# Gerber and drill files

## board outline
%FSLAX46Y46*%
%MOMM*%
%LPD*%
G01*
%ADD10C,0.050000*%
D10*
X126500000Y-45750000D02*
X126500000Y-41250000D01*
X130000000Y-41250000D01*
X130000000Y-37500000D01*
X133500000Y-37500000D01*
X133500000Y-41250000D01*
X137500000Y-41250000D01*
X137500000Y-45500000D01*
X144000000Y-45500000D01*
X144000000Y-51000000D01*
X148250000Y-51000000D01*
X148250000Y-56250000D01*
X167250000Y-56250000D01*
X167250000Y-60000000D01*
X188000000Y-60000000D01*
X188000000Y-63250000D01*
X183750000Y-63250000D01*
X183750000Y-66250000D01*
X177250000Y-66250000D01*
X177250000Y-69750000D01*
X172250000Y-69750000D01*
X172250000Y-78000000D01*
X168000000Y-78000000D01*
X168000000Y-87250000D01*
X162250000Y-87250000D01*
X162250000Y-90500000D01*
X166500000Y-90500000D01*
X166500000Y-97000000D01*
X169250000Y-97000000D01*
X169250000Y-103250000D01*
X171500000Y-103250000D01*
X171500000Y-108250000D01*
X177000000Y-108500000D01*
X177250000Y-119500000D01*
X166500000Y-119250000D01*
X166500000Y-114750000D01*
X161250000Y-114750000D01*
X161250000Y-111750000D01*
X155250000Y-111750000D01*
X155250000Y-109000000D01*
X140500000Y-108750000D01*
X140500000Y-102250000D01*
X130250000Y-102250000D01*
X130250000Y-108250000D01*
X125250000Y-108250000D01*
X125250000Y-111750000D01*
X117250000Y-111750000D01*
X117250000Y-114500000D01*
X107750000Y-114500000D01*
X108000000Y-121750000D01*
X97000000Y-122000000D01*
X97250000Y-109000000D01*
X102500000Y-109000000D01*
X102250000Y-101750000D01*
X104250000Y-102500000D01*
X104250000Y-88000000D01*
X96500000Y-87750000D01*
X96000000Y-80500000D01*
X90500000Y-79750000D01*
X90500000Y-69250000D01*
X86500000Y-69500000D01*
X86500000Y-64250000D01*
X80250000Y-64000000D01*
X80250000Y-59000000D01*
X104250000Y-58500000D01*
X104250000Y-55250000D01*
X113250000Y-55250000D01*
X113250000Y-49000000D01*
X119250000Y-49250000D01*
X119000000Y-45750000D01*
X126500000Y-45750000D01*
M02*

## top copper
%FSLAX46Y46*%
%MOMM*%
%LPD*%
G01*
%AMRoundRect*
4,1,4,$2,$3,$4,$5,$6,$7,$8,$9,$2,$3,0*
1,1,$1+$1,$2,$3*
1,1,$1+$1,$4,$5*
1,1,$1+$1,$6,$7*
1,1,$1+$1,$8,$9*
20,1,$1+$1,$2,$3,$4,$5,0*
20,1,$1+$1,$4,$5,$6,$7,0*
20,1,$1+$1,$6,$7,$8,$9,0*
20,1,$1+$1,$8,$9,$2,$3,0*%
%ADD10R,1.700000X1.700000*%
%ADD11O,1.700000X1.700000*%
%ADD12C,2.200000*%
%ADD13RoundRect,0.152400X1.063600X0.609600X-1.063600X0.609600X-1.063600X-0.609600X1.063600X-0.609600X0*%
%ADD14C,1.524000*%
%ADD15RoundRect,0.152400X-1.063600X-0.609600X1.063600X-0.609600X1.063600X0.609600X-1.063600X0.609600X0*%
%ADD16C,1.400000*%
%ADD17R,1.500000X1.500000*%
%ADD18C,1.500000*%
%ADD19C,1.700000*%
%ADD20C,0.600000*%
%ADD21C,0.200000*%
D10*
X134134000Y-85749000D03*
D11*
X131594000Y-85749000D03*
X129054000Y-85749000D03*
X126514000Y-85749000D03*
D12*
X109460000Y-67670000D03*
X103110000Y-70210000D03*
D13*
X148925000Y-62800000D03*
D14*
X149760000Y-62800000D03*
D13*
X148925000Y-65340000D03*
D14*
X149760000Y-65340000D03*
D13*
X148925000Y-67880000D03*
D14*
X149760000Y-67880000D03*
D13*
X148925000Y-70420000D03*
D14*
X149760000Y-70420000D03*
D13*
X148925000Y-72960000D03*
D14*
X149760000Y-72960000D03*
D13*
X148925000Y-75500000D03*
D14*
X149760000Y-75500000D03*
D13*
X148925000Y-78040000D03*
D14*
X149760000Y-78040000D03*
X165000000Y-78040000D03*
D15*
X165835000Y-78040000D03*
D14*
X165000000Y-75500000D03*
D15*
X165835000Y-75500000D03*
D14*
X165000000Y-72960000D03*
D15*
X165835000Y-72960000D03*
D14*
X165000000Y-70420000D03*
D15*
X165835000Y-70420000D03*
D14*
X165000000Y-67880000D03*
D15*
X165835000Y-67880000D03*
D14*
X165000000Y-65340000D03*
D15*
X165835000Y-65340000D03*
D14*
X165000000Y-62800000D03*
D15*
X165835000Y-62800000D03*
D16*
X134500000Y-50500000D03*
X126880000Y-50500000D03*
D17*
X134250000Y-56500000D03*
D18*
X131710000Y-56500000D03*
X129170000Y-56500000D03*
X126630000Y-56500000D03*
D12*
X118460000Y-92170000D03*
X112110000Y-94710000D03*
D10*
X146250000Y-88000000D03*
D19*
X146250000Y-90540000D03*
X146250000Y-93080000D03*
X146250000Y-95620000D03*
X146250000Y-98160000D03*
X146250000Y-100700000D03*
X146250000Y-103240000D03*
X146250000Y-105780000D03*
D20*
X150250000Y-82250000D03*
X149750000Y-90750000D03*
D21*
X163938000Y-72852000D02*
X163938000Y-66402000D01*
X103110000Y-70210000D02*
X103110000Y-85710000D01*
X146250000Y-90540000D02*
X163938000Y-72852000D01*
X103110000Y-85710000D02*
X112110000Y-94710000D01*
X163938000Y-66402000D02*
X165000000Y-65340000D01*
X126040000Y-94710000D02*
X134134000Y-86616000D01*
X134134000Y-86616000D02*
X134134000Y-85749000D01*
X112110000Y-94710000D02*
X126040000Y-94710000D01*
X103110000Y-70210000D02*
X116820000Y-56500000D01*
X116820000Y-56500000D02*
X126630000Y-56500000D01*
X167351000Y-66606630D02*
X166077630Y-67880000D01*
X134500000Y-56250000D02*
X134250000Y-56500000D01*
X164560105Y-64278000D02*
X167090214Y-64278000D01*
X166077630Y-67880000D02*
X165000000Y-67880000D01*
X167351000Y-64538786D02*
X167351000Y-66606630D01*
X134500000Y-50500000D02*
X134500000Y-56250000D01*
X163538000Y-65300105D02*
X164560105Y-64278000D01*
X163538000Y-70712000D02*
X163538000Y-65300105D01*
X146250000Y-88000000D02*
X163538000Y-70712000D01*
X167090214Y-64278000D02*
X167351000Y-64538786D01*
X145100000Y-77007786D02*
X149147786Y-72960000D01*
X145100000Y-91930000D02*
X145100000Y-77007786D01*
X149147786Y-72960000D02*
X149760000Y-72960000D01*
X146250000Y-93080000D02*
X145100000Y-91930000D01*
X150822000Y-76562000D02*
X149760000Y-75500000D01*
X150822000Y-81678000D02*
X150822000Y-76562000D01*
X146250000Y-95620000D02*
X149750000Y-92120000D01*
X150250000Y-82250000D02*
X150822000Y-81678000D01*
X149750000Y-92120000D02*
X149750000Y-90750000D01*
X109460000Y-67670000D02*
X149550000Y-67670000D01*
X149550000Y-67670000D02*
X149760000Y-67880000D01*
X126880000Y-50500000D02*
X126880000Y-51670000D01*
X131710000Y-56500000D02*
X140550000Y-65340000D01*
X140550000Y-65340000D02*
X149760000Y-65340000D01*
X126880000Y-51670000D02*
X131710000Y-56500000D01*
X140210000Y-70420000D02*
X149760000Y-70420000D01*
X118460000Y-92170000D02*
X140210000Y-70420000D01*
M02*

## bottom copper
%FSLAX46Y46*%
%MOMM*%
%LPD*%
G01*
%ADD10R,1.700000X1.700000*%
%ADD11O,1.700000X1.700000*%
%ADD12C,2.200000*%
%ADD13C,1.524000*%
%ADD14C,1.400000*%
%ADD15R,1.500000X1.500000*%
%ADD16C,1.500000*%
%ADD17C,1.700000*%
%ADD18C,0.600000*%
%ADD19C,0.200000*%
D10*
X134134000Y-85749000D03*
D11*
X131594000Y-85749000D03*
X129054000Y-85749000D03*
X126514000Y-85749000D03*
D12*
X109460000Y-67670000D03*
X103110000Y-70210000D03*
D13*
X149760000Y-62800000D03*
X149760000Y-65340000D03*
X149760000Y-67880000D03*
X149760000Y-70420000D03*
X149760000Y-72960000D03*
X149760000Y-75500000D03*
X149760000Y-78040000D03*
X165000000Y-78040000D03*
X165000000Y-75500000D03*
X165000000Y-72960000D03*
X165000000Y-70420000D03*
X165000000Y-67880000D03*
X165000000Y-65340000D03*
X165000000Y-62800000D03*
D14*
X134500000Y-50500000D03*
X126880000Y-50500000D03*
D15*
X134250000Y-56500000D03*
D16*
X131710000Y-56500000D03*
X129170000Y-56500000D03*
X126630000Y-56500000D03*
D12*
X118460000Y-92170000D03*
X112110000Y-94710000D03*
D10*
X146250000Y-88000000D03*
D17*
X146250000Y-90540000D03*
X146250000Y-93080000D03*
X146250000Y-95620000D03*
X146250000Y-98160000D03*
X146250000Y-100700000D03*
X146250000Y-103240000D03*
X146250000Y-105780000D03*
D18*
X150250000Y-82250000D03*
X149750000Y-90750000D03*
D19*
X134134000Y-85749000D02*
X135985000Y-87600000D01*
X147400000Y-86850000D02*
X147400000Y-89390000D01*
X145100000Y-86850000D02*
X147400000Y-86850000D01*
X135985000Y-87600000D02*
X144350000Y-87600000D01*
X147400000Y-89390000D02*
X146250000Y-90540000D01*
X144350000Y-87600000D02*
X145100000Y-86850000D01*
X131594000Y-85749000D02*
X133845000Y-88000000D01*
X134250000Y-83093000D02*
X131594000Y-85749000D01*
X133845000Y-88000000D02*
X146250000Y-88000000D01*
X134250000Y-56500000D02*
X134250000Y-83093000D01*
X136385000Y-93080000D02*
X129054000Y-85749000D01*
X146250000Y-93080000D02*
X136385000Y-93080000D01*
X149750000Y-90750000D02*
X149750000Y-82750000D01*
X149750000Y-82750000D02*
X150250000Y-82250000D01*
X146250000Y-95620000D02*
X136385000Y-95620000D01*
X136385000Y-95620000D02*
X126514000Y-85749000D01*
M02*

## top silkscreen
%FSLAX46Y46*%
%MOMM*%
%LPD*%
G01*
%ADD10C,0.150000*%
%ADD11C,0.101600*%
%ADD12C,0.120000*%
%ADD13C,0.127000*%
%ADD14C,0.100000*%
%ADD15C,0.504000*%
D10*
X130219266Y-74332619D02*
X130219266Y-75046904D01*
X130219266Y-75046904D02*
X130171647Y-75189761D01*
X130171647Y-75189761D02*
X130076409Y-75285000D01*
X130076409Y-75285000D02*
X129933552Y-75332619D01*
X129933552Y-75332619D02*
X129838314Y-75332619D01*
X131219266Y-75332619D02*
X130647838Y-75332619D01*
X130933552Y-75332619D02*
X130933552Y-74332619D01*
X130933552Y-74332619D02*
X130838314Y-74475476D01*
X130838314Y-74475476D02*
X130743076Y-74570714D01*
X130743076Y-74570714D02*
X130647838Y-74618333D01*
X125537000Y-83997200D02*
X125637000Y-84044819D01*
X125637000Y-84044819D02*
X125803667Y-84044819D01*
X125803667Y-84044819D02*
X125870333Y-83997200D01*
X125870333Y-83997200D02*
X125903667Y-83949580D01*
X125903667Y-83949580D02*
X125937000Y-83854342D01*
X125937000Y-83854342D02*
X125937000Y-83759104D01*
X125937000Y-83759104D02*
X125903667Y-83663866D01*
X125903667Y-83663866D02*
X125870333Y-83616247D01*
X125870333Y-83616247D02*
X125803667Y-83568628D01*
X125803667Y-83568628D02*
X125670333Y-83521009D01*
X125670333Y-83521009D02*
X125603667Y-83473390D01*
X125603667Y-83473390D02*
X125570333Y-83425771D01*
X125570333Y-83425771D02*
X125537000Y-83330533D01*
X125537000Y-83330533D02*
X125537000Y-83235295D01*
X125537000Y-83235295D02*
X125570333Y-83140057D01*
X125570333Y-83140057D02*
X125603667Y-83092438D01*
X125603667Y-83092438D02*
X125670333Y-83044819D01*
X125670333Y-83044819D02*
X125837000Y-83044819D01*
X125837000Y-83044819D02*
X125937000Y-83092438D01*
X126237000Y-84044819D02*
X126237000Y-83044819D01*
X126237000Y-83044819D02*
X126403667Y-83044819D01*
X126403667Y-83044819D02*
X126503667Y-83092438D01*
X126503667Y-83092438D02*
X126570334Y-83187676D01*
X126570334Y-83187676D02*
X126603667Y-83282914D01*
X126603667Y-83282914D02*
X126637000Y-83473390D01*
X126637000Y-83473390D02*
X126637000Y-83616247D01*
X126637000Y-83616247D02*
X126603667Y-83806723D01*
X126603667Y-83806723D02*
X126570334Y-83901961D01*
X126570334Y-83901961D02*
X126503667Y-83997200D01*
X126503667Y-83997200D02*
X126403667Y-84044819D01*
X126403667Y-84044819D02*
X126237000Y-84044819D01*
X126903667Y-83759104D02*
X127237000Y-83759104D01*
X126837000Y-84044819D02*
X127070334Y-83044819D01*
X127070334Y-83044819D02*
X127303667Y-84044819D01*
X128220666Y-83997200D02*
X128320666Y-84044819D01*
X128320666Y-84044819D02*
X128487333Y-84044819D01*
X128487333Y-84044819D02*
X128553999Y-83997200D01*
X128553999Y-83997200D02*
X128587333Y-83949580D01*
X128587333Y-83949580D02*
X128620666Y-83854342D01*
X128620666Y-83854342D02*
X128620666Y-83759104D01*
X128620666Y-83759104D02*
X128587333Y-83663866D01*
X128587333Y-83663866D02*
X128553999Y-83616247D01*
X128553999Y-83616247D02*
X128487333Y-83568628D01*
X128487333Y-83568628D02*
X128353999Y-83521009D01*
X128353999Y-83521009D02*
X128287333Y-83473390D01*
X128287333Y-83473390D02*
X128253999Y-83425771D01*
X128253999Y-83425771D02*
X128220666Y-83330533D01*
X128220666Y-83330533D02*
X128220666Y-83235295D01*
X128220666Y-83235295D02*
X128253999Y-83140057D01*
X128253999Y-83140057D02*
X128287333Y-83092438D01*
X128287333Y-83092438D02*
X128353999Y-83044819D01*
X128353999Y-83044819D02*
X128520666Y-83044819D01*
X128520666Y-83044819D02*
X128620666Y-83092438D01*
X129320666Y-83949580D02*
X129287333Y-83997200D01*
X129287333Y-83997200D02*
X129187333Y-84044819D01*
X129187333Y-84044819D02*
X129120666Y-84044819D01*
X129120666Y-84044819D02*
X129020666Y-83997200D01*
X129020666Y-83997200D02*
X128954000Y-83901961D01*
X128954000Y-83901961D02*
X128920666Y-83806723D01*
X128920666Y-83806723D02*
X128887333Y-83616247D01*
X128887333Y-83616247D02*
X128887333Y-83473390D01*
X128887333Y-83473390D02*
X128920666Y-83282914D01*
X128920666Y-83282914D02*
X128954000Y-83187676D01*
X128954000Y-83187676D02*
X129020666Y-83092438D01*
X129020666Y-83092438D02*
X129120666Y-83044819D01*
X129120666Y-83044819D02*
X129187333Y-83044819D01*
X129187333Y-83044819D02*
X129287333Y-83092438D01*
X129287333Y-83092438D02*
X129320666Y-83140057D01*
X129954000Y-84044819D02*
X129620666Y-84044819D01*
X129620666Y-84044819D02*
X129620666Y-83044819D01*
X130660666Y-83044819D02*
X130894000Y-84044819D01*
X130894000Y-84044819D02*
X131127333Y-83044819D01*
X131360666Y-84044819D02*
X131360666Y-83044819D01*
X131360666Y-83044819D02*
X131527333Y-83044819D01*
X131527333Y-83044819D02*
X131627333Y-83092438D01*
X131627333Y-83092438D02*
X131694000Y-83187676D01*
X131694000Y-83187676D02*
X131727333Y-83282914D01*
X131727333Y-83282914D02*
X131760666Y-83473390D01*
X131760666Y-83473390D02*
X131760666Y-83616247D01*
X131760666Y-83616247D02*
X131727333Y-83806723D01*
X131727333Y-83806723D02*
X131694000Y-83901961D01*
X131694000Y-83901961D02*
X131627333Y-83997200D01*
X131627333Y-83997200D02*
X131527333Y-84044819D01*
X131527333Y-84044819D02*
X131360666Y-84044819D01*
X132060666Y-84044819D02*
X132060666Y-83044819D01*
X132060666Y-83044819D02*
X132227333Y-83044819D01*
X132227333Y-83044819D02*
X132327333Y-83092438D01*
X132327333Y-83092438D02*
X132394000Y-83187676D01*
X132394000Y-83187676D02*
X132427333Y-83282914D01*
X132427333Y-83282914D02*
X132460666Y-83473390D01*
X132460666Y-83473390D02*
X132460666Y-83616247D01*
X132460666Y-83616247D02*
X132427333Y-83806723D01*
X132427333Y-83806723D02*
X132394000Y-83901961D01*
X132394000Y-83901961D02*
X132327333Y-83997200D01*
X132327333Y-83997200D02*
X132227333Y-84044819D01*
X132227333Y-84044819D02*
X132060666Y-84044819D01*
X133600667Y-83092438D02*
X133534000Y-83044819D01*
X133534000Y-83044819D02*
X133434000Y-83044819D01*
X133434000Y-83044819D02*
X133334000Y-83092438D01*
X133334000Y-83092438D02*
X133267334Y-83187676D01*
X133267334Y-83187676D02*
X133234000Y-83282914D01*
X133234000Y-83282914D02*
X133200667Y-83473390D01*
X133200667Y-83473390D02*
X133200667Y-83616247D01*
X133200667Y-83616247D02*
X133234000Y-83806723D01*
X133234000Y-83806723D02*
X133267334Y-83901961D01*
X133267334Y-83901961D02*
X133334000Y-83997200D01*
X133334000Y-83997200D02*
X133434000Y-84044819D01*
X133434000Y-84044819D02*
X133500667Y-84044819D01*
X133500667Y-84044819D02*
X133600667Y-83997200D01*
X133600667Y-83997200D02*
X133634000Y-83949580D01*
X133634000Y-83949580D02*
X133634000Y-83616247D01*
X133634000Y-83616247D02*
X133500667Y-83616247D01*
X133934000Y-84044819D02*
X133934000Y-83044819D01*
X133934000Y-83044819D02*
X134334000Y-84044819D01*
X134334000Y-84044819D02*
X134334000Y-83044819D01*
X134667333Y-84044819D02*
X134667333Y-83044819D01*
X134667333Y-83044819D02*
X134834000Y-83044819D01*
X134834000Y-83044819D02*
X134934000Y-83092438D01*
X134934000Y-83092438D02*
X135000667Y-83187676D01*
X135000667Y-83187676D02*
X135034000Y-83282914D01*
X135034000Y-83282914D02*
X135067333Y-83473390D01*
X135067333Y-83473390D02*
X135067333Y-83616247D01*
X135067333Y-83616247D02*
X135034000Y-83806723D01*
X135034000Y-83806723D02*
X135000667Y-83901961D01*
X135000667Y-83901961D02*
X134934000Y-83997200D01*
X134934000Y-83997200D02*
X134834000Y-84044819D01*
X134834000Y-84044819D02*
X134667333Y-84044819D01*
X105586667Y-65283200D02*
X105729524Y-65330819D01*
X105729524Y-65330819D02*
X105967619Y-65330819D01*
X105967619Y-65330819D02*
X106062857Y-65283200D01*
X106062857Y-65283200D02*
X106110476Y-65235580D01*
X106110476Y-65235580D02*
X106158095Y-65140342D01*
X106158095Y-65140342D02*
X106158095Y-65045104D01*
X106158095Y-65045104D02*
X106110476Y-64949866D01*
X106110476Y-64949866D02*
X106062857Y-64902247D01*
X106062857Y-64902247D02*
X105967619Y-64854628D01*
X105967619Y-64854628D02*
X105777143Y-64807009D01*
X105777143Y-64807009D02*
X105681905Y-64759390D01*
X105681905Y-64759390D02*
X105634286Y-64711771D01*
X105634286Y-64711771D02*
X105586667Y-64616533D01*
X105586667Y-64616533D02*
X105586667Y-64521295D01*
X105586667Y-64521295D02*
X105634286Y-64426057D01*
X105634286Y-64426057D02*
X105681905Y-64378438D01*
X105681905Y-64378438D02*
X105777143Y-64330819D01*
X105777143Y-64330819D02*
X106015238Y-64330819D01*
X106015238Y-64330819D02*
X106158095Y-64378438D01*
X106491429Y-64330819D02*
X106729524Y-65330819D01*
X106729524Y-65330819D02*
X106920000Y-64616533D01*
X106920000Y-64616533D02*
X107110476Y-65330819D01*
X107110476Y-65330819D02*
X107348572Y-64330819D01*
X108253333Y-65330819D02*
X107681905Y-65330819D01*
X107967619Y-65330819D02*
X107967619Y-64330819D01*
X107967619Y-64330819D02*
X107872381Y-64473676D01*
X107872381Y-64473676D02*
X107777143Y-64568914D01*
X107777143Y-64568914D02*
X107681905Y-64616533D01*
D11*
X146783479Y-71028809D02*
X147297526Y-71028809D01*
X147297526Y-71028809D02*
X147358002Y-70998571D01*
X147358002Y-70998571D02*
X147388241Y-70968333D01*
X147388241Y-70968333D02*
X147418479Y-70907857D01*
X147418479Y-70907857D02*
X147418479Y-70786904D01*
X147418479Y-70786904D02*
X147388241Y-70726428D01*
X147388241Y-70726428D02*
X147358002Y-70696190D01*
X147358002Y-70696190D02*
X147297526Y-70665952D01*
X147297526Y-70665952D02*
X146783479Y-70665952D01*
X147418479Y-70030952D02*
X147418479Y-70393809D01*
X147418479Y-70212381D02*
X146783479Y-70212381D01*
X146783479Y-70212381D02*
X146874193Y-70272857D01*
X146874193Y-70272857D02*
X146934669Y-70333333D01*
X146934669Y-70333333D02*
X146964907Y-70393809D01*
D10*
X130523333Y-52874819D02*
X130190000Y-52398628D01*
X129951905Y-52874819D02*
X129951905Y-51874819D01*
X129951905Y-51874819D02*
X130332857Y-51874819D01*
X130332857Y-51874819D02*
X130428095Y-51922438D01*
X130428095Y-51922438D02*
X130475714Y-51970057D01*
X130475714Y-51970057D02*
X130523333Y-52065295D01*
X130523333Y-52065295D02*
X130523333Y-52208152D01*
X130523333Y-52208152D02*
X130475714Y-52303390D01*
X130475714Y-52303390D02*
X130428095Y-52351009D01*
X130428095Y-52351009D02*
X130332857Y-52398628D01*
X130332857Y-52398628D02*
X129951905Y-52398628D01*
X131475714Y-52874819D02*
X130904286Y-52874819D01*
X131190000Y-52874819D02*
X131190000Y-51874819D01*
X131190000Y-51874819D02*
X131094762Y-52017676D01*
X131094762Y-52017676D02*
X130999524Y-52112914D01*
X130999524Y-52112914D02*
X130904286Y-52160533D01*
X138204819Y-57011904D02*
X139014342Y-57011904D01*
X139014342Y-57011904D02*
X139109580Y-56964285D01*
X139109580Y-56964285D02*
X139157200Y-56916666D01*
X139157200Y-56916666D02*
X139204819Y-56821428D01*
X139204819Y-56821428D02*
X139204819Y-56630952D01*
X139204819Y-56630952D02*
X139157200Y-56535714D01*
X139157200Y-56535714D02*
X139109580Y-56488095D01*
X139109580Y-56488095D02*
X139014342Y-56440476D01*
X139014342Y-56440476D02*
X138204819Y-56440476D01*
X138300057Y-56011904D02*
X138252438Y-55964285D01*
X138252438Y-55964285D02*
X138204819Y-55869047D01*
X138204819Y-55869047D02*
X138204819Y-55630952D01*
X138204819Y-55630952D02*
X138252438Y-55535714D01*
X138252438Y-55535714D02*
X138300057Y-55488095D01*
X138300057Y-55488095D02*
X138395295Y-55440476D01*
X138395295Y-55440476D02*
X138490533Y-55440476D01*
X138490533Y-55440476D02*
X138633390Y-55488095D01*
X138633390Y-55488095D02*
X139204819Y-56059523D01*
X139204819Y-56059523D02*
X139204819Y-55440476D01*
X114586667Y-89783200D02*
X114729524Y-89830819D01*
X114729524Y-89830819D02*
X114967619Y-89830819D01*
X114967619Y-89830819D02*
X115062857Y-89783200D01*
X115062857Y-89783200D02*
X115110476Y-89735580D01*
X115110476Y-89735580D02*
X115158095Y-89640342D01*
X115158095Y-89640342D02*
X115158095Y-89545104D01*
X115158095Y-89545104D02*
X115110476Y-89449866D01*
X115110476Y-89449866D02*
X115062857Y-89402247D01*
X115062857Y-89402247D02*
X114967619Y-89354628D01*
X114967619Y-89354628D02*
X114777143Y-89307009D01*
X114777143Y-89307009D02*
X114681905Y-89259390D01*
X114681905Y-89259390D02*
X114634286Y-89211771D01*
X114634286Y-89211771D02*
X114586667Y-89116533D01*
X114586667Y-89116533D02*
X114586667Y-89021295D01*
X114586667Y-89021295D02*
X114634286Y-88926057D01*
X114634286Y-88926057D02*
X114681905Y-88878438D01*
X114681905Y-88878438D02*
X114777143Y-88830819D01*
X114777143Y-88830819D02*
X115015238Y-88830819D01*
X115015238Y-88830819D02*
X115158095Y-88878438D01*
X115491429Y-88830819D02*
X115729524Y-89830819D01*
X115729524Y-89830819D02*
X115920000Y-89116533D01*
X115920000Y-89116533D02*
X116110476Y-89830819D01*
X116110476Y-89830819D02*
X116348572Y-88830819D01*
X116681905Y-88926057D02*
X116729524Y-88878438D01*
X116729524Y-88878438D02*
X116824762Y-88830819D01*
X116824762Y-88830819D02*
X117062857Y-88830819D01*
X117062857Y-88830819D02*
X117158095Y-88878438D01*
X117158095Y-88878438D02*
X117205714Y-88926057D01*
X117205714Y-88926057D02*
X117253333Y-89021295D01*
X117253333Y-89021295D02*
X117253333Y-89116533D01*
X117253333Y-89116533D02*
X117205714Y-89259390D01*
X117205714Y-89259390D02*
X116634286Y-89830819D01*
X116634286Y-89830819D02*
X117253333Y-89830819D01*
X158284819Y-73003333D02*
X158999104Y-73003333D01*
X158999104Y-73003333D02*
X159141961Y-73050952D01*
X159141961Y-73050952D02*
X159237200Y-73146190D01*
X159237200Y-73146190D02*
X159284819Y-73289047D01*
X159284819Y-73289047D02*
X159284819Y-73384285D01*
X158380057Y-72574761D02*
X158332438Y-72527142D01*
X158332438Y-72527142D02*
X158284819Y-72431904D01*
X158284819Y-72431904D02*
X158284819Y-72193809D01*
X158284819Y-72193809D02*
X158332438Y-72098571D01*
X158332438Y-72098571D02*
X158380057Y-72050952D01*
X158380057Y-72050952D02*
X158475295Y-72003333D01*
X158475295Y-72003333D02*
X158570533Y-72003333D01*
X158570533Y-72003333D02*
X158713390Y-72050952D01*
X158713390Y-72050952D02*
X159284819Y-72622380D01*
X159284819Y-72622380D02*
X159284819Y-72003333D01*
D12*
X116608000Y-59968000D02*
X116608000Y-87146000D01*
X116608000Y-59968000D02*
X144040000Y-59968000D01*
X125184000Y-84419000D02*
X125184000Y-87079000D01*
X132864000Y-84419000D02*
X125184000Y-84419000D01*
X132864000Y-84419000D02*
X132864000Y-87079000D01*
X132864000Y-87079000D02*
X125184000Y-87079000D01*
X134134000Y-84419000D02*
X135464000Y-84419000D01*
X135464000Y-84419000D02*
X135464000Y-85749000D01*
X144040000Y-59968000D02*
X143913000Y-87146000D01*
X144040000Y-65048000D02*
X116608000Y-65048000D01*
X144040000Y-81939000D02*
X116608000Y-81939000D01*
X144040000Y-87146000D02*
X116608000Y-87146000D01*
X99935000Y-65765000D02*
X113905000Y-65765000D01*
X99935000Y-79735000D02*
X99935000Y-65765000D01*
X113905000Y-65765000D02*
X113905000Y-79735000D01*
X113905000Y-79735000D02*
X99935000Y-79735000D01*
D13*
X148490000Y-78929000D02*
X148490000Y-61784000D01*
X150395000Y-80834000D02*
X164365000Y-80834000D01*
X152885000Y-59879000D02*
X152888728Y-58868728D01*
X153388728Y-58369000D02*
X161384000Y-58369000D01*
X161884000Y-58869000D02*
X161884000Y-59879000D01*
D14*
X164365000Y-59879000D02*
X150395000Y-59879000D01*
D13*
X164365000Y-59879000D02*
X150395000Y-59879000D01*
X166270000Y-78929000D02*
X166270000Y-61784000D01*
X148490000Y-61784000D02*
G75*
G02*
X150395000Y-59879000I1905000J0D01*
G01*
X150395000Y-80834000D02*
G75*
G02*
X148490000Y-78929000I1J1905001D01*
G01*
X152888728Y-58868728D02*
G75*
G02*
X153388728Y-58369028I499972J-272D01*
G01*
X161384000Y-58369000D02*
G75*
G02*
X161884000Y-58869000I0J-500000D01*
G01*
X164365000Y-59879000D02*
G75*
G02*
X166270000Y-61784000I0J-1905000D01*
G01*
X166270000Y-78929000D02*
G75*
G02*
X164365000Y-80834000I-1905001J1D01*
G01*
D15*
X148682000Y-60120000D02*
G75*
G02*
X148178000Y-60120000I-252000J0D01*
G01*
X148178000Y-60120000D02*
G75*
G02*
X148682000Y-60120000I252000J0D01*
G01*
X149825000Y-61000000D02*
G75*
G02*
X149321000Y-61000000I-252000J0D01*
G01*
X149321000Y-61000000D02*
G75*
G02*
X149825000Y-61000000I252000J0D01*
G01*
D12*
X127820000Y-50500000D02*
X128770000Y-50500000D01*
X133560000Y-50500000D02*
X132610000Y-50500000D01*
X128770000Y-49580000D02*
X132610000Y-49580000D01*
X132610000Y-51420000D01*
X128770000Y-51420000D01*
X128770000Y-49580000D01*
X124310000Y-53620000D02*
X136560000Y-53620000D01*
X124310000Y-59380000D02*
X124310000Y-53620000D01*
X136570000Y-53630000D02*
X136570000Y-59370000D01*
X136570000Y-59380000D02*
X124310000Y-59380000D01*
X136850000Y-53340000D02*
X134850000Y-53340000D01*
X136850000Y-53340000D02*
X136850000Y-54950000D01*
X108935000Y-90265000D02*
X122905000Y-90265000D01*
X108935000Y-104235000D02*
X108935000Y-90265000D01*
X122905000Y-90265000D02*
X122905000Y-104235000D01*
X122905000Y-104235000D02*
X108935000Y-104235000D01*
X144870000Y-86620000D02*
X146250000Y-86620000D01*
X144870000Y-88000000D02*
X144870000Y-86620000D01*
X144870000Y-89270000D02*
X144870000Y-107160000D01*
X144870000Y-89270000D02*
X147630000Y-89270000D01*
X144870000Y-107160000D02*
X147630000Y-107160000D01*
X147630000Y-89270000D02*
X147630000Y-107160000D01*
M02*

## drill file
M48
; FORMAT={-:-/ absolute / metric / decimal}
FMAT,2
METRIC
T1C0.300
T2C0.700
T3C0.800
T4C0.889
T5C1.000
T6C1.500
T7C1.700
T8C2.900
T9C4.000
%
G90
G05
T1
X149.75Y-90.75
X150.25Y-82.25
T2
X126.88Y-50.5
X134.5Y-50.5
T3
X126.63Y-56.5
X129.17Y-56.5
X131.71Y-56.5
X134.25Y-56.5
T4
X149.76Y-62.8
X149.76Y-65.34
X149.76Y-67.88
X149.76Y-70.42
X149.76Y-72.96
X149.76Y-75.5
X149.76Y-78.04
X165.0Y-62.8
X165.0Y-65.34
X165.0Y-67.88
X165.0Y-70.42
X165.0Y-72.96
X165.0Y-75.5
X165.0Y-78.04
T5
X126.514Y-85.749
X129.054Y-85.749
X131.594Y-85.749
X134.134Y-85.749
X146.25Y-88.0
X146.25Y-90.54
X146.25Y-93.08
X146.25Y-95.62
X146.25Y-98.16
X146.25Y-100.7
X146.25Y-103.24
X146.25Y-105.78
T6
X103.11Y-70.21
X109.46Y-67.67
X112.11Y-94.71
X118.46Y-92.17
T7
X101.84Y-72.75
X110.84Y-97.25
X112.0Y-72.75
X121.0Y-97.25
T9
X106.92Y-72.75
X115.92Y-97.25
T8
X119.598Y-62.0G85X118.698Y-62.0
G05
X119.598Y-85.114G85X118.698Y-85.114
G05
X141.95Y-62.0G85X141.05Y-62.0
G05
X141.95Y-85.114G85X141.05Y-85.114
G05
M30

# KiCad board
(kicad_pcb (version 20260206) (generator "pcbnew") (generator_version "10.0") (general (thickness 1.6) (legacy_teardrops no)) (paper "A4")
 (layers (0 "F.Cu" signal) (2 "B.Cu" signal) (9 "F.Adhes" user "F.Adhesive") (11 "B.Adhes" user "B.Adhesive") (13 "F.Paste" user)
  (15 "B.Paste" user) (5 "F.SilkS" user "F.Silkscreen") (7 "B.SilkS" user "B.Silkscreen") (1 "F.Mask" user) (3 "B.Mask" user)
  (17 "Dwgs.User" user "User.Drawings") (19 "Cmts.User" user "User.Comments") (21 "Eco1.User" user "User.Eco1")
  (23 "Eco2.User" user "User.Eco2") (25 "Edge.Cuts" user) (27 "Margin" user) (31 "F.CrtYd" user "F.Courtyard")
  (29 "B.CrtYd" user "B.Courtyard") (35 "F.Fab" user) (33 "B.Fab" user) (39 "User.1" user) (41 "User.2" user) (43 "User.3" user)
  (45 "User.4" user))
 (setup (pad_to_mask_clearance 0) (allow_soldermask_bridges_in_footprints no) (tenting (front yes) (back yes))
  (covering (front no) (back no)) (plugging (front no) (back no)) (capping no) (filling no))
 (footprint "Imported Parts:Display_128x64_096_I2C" (layer "F.Cu") (at 130.324 85.749 180)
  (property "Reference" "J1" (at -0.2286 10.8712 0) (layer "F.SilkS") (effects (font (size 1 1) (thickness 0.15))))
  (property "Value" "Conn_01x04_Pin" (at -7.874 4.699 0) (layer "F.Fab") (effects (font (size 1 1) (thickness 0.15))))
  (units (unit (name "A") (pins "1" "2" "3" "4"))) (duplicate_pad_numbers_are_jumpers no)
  (fp_line (start 13.716 25.781) (end 13.716 -1.397) (stroke (width 0.12) (type solid)) (layer "F.SilkS"))
  (fp_line (start 13.716 25.781) (end -13.716 25.781) (stroke (width 0.12) (type solid)) (layer "F.SilkS"))
  (fp_line (start 5.14 1.33) (end 5.14 -1.33) (stroke (width 0.12) (type solid)) (layer "F.SilkS"))
  (fp_line (start -2.54 1.33) (end 5.14 1.33) (stroke (width 0.12) (type solid)) (layer "F.SilkS"))
  (fp_line (start -2.54 1.33) (end -2.54 -1.33) (stroke (width 0.12) (type solid)) (layer "F.SilkS"))
  (fp_line (start -2.54 -1.33) (end 5.14 -1.33) (stroke (width 0.12) (type solid)) (layer "F.SilkS"))
  (fp_line (start -3.81 1.33) (end -5.14 1.33) (stroke (width 0.12) (type solid)) (layer "F.SilkS"))
  (fp_line (start -5.14 1.33) (end -5.14 0) (stroke (width 0.12) (type solid)) (layer "F.SilkS"))
  (fp_line (start -13.716 25.781) (end -13.589 -1.397) (stroke (width 0.12) (type solid)) (layer "F.SilkS"))
  (fp_line (start -13.716 20.701) (end 13.716 20.701) (stroke (width 0.12) (type solid)) (layer "F.SilkS"))
  (fp_line (start -13.716 3.81) (end 13.716 3.81) (stroke (width 0.12) (type solid)) (layer "F.SilkS"))
  (fp_line (start -13.716 -1.397) (end 13.716 -1.397) (stroke (width 0.12) (type solid)) (layer "F.SilkS"))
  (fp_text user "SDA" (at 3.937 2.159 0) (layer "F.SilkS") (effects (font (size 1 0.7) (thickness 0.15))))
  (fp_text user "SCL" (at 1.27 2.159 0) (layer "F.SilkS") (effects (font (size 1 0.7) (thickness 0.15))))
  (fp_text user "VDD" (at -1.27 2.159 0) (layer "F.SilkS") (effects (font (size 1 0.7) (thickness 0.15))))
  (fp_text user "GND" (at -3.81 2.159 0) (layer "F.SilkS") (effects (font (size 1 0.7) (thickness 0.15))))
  (pad "" np_thru_hole oval (at -11.176 0.635 180) (size 3.8 2.9) (drill oval 3.8 2.9) (layers "*.Cu" "*.Mask"))
  (pad "" np_thru_hole oval (at -11.176 23.749 180) (size 3.8 2.9) (drill oval 3.8 2.9) (layers "*.Cu" "*.Mask"))
  (pad "" np_thru_hole oval (at 11.176 0.635 180) (size 3.8 2.9) (drill oval 3.8 2.9) (layers "*.Cu" "*.Mask"))
  (pad "" np_thru_hole oval (at 11.176 23.749 180) (size 3.8 2.9) (drill oval 3.8 2.9) (layers "*.Cu" "*.Mask"))
  (pad "1" thru_hole rect (at -3.81 0 270) (size 1.7 1.7) (drill 1) (layers "*.Cu" "*.Mask") (remove_unused_layers no) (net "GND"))
  (pad "2" thru_hole oval (at -1.27 0 270) (size 1.7 1.7) (drill 1) (layers "*.Cu" "*.Mask") (remove_unused_layers no) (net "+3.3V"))
  (pad "3" thru_hole oval (at 1.27 0 270) (size 1.7 1.7) (drill 1) (layers "*.Cu" "*.Mask") (remove_unused_layers no) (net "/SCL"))
  (pad "4" thru_hole oval (at 3.81 0 270) (size 1.7 1.7) (drill 1) (layers "*.Cu" "*.Mask") (remove_unused_layers no) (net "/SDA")))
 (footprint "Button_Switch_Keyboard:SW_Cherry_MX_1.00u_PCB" (layer "F.Cu") (at 109.46 67.67)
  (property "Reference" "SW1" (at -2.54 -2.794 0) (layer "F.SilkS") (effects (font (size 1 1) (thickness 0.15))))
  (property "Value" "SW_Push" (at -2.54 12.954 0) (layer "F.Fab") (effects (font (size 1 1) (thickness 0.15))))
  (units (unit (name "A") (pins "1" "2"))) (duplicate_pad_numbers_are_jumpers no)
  (fp_line (start -9.525 -1.905) (end 4.445 -1.905) (stroke (width 0.12) (type solid)) (layer "F.SilkS"))
  (fp_line (start -9.525 12.065) (end -9.525 -1.905) (stroke (width 0.12) (type solid)) (layer "F.SilkS"))
  (fp_line (start 4.445 -1.905) (end 4.445 12.065) (stroke (width 0.12) (type solid)) (layer "F.SilkS"))
  (fp_line (start 4.445 12.065) (end -9.525 12.065) (stroke (width 0.12) (type solid)) (layer "F.SilkS"))
  (pad "" np_thru_hole circle (at -7.62 5.08) (size 1.7 1.7) (drill 1.7) (layers "*.Cu" "*.Mask"))
  (pad "" np_thru_hole circle (at -2.54 5.08) (size 4 4) (drill 4) (layers "*.Cu" "*.Mask"))
  (pad "" np_thru_hole circle (at 2.54 5.08) (size 1.7 1.7) (drill 1.7) (layers "*.Cu" "*.Mask"))
  (pad "1" thru_hole circle (at 0 0) (size 2.2 2.2) (drill 1.5) (layers "*.Cu" "*.Mask") (remove_unused_layers no) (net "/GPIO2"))
  (pad "2" thru_hole circle (at -6.35 2.54) (size 2.2 2.2) (drill 1.5) (layers "*.Cu" "*.Mask") (remove_unused_layers no) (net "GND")))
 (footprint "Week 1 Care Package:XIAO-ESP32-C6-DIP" (layer "F.Cu") (at 157.38 70.42 90)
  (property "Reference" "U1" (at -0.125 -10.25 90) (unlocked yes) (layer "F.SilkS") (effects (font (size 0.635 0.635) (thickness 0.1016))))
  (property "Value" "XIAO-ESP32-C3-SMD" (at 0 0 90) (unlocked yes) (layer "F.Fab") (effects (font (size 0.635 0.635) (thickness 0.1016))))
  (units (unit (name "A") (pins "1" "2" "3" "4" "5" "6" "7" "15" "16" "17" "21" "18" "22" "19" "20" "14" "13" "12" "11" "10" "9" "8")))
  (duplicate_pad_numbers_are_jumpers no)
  (fp_line (start -8.509 -8.89) (end 8.636 -8.89) (stroke (width 0.127) (type solid)) (layer "F.SilkS"))
  (fp_line (start -10.414 -6.985) (end -10.414 6.985) (stroke (width 0.127) (type solid)) (layer "F.SilkS"))
  (fp_line (start 10.541 -4.495) (end 11.551272 -4.491272) (stroke (width 0.127) (type solid)) (layer "F.SilkS"))
  (fp_line (start 12.051 -3.991272) (end 12.051 4.004) (stroke (width 0.127) (type solid)) (layer "F.SilkS"))
  (fp_line (start 11.551 4.504) (end 10.541 4.504) (stroke (width 0.127) (type solid)) (layer "F.SilkS"))
  (fp_line (start 10.541 6.985) (end 10.541 -6.985) (stroke (width 0.1) (type solid)) (layer "F.SilkS"))
  (fp_line (start 10.541 6.985) (end 10.541 -6.985) (stroke (width 0.127) (type solid)) (layer "F.SilkS"))
  (fp_line (start -8.509 8.89) (end 8.636 8.89) (stroke (width 0.127) (type solid)) (layer "F.SilkS"))
  (fp_arc (start 8.636 -8.89) (mid 9.983038 -8.332038) (end 10.541 -6.985) (stroke (width 0.127) (type solid)) (layer "F.SilkS"))
  (fp_arc (start -10.414 -6.985) (mid -9.856038 -8.332038) (end -8.509 -8.89) (stroke (width 0.127) (type solid)) (layer "F.SilkS"))
  (fp_arc (start 11.551272 -4.491272) (mid 11.904644 -4.344724) (end 12.051 -3.991272) (stroke (width 0.127) (type default))
   (layer "F.SilkS"))
  (fp_arc (start 12.051 4.004) (mid 11.904553 4.357553) (end 11.551 4.504) (stroke (width 0.127) (type default)) (layer "F.SilkS"))
  (fp_arc (start 10.541 6.985) (mid 9.983038 8.332038) (end 8.636 8.89) (stroke (width 0.127) (type solid)) (layer "F.SilkS"))
  (fp_arc (start -8.509 8.89) (mid -9.856038 8.332038) (end -10.414 6.985) (stroke (width 0.127) (type solid)) (layer "F.SilkS"))
  (fp_circle (center 10.3 -8.95) (end 10.554 -8.95) (stroke (width 0.5) (type solid)) (fill yes) (layer "F.SilkS"))
  (fp_circle (center 9.42 -7.807) (end 9.674 -7.807) (stroke (width 0.5) (type solid)) (fill yes) (layer "F.SilkS"))
  (pad "1" smd roundrect (at 7.62 -8.455 180) (size 2.432 1.524) (layers "F.Cu" "F.Mask") (roundrect_rratio 0.1)
   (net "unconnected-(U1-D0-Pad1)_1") (thermal_bridge_angle 45))
  (pad "1" thru_hole circle (at 7.62 -7.62 180) (size 1.524 1.524) (drill 0.889) (layers "*.Cu" "*.Mask") (remove_unused_layers no)
   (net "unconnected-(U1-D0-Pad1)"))
  (pad "2" smd roundrect (at 5.08 -8.455 180) (size 2.432 1.524) (layers "F.Cu" "F.Mask") (roundrect_rratio 0.1) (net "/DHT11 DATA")
   (thermal_bridge_angle 45))
  (pad "2" thru_hole circle (at 5.08 -7.62 180) (size 1.524 1.524) (drill 0.889) (layers "*.Cu" "*.Mask") (remove_unused_layers no)
   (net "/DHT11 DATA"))
  (pad "3" smd roundrect (at 2.54 -8.455 180) (size 2.432 1.524) (layers "F.Cu" "F.Mask") (roundrect_rratio 0.1) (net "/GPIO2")
   (thermal_bridge_angle 45))
  (pad "3" thru_hole circle (at 2.54 -7.62 180) (size 1.524 1.524) (drill 0.889) (layers "*.Cu" "*.Mask") (remove_unused_layers no)
   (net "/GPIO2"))
  (pad "4" smd roundrect (at 0 -8.455 180) (size 2.432 1.524) (layers "F.Cu" "F.Mask") (roundrect_rratio 0.1) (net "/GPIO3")
   (thermal_bridge_angle 45))
  (pad "4" thru_hole circle (at 0 -7.62 180) (size 1.524 1.524) (drill 0.889) (layers "*.Cu" "*.Mask") (remove_unused_layers no)
   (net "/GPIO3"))
  (pad "5" smd roundrect (at -2.54 -8.455 180) (size 2.432 1.524) (layers "F.Cu" "F.Mask") (roundrect_rratio 0.1) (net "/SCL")
   (thermal_bridge_angle 45))
  (pad "5" thru_hole circle (at -2.54 -7.62 180) (size 1.524 1.524) (drill 0.889) (layers "*.Cu" "*.Mask") (remove_unused_layers no)
   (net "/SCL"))
  (pad "6" smd roundrect (at -5.08 -8.455 180) (size 2.432 1.524) (layers "F.Cu" "F.Mask") (roundrect_rratio 0.1) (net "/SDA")
   (thermal_bridge_angle 45))
  (pad "6" thru_hole circle (at -5.08 -7.62 180) (size 1.524 1.524) (drill 0.889) (layers "*.Cu" "*.Mask") (remove_unused_layers no)
   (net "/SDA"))
  (pad "7" smd roundrect (at -7.62 -8.455 180) (size 2.432 1.524) (layers "F.Cu" "F.Mask") (roundrect_rratio 0.1)
   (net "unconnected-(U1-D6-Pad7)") (thermal_bridge_angle 45))
  (pad "7" thru_hole circle (at -7.62 -7.62 180) (size 1.524 1.524) (drill 0.889) (layers "*.Cu" "*.Mask") (remove_unused_layers no)
   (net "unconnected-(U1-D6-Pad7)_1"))
  (pad "8" thru_hole circle (at -7.62 7.62) (size 1.524 1.524) (drill 0.889) (layers "*.Cu" "*.Mask") (remove_unused_layers no)
   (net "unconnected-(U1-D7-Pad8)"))
  (pad "8" smd roundrect (at -7.62 8.455) (size 2.432 1.524) (layers "F.Cu" "F.Mask") (roundrect_rratio 0.1)
   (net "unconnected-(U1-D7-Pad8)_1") (thermal_bridge_angle 45))
  (pad "9" thru_hole circle (at -5.08 7.62) (size 1.524 1.524) (drill 0.889) (layers "*.Cu" "*.Mask") (remove_unused_layers no)
   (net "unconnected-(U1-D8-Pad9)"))
  (pad "9" smd roundrect (at -5.08 8.455) (size 2.432 1.524) (layers "F.Cu" "F.Mask") (roundrect_rratio 0.1)
   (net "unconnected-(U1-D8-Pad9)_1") (thermal_bridge_angle 45))
  (pad "10" thru_hole circle (at -2.54 7.62) (size 1.524 1.524) (drill 0.889) (layers "*.Cu" "*.Mask") (remove_unused_layers no)
   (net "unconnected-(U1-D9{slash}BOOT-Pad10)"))
  (pad "10" smd roundrect (at -2.54 8.455) (size 2.432 1.524) (layers "F.Cu" "F.Mask") (roundrect_rratio 0.1)
   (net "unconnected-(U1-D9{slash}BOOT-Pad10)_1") (thermal_bridge_angle 45))
  (pad "11" thru_hole circle (at 0 7.62) (size 1.524 1.524) (drill 0.889) (layers "*.Cu" "*.Mask") (remove_unused_layers no)
   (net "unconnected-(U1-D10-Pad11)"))
  (pad "11" smd roundrect (at 0 8.455) (size 2.432 1.524) (layers "F.Cu" "F.Mask") (roundrect_rratio 0.1)
   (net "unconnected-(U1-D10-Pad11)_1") (thermal_bridge_angle 45))
  (pad "12" thru_hole circle (at 2.54 7.62) (size 1.524 1.524) (drill 0.889) (layers "*.Cu" "*.Mask") (remove_unused_layers no)
   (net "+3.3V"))
  (pad "12" smd roundrect (at 2.54 8.455) (size 2.432 1.524) (layers "F.Cu" "F.Mask") (roundrect_rratio 0.1) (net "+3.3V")
   (thermal_bridge_angle 45))
  (pad "13" thru_hole circle (at 5.08 7.62) (size 1.524 1.524) (drill 0.889) (layers "*.Cu" "*.Mask") (remove_unused_layers no) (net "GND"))
  (pad "13" smd roundrect (at 5.08 8.455) (size 2.432 1.524) (layers "F.Cu" "F.Mask") (roundrect_rratio 0.1) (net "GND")
   (thermal_bridge_angle 45))
  (pad "14" thru_hole circle (at 7.62 7.62) (size 1.524 1.524) (drill 0.889) (layers "*.Cu" "*.Mask") (remove_unused_layers no) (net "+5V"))
  (pad "14" smd roundrect (at 7.62 8.455) (size 2.432 1.524) (layers "F.Cu" "F.Mask") (roundrect_rratio 0.1) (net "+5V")
   (thermal_bridge_angle 45)))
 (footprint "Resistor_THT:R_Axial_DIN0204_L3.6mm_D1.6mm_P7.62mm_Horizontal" (layer "F.Cu") (at 134.5 50.5 180)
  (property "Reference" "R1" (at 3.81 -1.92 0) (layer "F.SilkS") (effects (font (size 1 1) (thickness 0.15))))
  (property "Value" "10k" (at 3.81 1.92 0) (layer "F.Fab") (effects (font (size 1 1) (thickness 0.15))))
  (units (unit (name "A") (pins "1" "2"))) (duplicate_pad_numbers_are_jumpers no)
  (fp_line (start 6.68 0) (end 5.73 0) (stroke (width 0.12) (type solid)) (layer "F.SilkS"))
  (fp_line (start 0.94 0) (end 1.89 0) (stroke (width 0.12) (type solid)) (layer "F.SilkS"))
  (fp_rect (start 1.89 -0.92) (end 5.73 0.92) (stroke (width 0.12) (type solid)) (fill no) (layer "F.SilkS"))
  (pad "1" thru_hole circle (at 0 0 180) (size 1.4 1.4) (drill 0.7) (layers "*.Cu" "*.Mask") (remove_unused_layers no) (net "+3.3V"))
  (pad "2" thru_hole circle (at 7.62 0 180) (size 1.4 1.4) (drill 0.7) (layers "*.Cu" "*.Mask") (remove_unused_layers no)
   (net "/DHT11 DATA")))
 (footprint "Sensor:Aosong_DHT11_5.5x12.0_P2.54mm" (layer "F.Cu") (at 134.25 56.5 -90)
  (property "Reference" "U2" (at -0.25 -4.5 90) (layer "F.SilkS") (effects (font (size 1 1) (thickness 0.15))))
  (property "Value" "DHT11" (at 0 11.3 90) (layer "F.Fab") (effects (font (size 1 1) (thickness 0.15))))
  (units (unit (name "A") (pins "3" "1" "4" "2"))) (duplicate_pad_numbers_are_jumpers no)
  (fp_line (start -2.88 9.94) (end -2.88 -2.31) (stroke (width 0.12) (type solid)) (layer "F.SilkS"))
  (fp_line (start 2.88 9.94) (end -2.88 9.94) (stroke (width 0.12) (type solid)) (layer "F.SilkS"))
  (fp_line (start -2.87 -2.32) (end 2.87 -2.32) (stroke (width 0.12) (type solid)) (layer "F.SilkS"))
  (fp_line (start 2.88 -2.32) (end 2.88 9.94) (stroke (width 0.12) (type solid)) (layer "F.SilkS"))
  (fp_line (start -3.16 -2.6) (end -3.16 -0.6) (stroke (width 0.12) (type solid)) (layer "F.SilkS"))
  (fp_line (start -3.16 -2.6) (end -1.55 -2.6) (stroke (width 0.12) (type solid)) (layer "F.SilkS"))
  (pad "1" thru_hole rect (at 0 0 270) (size 1.5 1.5) (drill 0.8) (layers "*.Cu" "*.Mask") (remove_unused_layers no) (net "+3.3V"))
  (pad "2" thru_hole circle (at 0 2.54 270) (size 1.5 1.5) (drill 0.8) (layers "*.Cu" "*.Mask") (remove_unused_layers no)
   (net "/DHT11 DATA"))
  (pad "3" thru_hole circle (at 0 5.08 270) (size 1.5 1.5) (drill 0.8) (layers "*.Cu" "*.Mask") (remove_unused_layers no)
   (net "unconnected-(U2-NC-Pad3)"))
  (pad "4" thru_hole circle (at 0 7.62 270) (size 1.5 1.5) (drill 0.8) (layers "*.Cu" "*.Mask") (remove_unused_layers no) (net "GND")))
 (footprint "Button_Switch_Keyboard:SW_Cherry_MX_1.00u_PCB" (layer "F.Cu") (at 118.46 92.17)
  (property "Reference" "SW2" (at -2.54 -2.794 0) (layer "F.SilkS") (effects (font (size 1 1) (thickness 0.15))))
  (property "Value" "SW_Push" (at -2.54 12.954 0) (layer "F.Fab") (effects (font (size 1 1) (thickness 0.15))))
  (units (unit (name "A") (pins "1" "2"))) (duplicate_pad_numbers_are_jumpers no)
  (fp_line (start -9.525 -1.905) (end 4.445 -1.905) (stroke (width 0.12) (type solid)) (layer "F.SilkS"))
  (fp_line (start -9.525 12.065) (end -9.525 -1.905) (stroke (width 0.12) (type solid)) (layer "F.SilkS"))
  (fp_line (start 4.445 -1.905) (end 4.445 12.065) (stroke (width 0.12) (type solid)) (layer "F.SilkS"))
  (fp_line (start 4.445 12.065) (end -9.525 12.065) (stroke (width 0.12) (type solid)) (layer "F.SilkS"))
  (pad "" np_thru_hole circle (at -7.62 5.08) (size 1.7 1.7) (drill 1.7) (layers "*.Cu" "*.Mask"))
  (pad "" np_thru_hole circle (at -2.54 5.08) (size 4 4) (drill 4) (layers "*.Cu" "*.Mask"))
  (pad "" np_thru_hole circle (at 2.54 5.08) (size 1.7 1.7) (drill 1.7) (layers "*.Cu" "*.Mask"))
  (pad "1" thru_hole circle (at 0 0) (size 2.2 2.2) (drill 1.5) (layers "*.Cu" "*.Mask") (remove_unused_layers no) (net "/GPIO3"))
  (pad "2" thru_hole circle (at -6.35 2.54) (size 2.2 2.2) (drill 1.5) (layers "*.Cu" "*.Mask") (remove_unused_layers no) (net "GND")))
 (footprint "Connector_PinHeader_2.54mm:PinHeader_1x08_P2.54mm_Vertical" (layer "F.Cu") (at 146.25 88)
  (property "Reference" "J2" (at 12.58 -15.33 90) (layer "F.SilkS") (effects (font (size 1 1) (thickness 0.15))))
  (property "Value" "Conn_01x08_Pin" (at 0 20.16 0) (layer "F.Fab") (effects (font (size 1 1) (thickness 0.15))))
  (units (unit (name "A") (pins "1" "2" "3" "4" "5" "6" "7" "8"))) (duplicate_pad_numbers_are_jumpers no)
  (fp_line (start -1.38 -1.38) (end 0 -1.38) (stroke (width 0.12) (type solid)) (layer "F.SilkS"))
  (fp_line (start -1.38 0) (end -1.38 -1.38) (stroke (width 0.12) (type solid)) (layer "F.SilkS"))
  (fp_line (start -1.38 1.27) (end -1.38 19.16) (stroke (width 0.12) (type solid)) (layer "F.SilkS"))
  (fp_line (start -1.38 1.27) (end 1.38 1.27) (stroke (width 0.12) (type solid)) (layer "F.SilkS"))
  (fp_line (start -1.38 19.16) (end 1.38 19.16) (stroke (width 0.12) (type solid)) (layer "F.SilkS"))
  (fp_line (start 1.38 1.27) (end 1.38 19.16) (stroke (width 0.12) (type solid)) (layer "F.SilkS"))
  (pad "1" thru_hole rect (at 0 0) (size 1.7 1.7) (drill 1) (layers "*.Cu" "*.Mask") (remove_unused_layers no) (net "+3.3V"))
  (pad "2" thru_hole circle (at 0 2.54) (size 1.7 1.7) (drill 1) (layers "*.Cu" "*.Mask") (remove_unused_layers no) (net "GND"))
  (pad "3" thru_hole circle (at 0 5.08) (size 1.7 1.7) (drill 1) (layers "*.Cu" "*.Mask") (remove_unused_layers no) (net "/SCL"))
  (pad "4" thru_hole circle (at 0 7.62) (size 1.7 1.7) (drill 1) (layers "*.Cu" "*.Mask") (remove_unused_layers no) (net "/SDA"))
  (pad "5" thru_hole circle (at 0 10.16) (size 1.7 1.7) (drill 1) (layers "*.Cu" "*.Mask") (remove_unused_layers no)
   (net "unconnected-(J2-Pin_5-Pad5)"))
  (pad "6" thru_hole circle (at 0 12.7) (size 1.7 1.7) (drill 1) (layers "*.Cu" "*.Mask") (remove_unused_layers no)
   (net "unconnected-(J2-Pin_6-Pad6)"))
  (pad "7" thru_hole circle (at 0 15.24) (size 1.7 1.7) (drill 1) (layers "*.Cu" "*.Mask") (remove_unused_layers no)
   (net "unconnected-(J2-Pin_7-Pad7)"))
  (pad "8" thru_hole circle (at 0 17.78) (size 1.7 1.7) (drill 1) (layers "*.Cu" "*.Mask") (remove_unused_layers no)
   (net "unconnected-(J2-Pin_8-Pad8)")))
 (gr_poly
  (pts (xy 126.5 45.75) (xy 126.5 41.25) (xy 130 41.25) (xy 130 37.5) (xy 133.5 37.5) (xy 133.5 41.25) (xy 137.5 41.25) (xy 137.5 45.5)
   (xy 144 45.5) (xy 144 51) (xy 148.25 51) (xy 148.25 56.25) (xy 167.25 56.25) (xy 167.25 60) (xy 188 60) (xy 188 63.25) (xy 183.75 63.25)
   (xy 183.75 66.25) (xy 177.25 66.25) (xy 177.25 69.75) (xy 172.25 69.75) (xy 172.25 78) (xy 168 78) (xy 168 87.25) (xy 162.25 87.25)
   (xy 162.25 90.5) (xy 166.5 90.5) (xy 166.5 97) (xy 169.25 97) (xy 169.25 103.25) (xy 171.5 103.25) (xy 171.5 108.25) (xy 177 108.5)
   (xy 177.25 119.5) (xy 166.5 119.25) (xy 166.5 114.75) (xy 161.25 114.75) (xy 161.25 111.75) (xy 155.25 111.75) (xy 155.25 109)
   (xy 140.5 108.75) (xy 140.5 102.25) (xy 130.25 102.25) (xy 130.25 108.25) (xy 125.25 108.25) (xy 125.25 111.75) (xy 117.25 111.75)
   (xy 117.25 114.5) (xy 107.75 114.5) (xy 108 121.75) (xy 97 122) (xy 97.25 109) (xy 102.5 109) (xy 102.25 101.75) (xy 104.25 102.5)
   (xy 104.25 88) (xy 96.5 87.75) (xy 96 80.5) (xy 90.5 79.75) (xy 90.5 69.25) (xy 86.5 69.5) (xy 86.5 64.25) (xy 80.25 64) (xy 80.25 59)
   (xy 104.25 58.5) (xy 104.25 55.25) (xy 113.25 55.25) (xy 113.25 49) (xy 119.25 49.25) (xy 119 45.75))
  (stroke (width 0.05) (type solid)) (fill no) (layer "Edge.Cuts"))
 (segment (start 163.938 72.852) (end 163.938 66.402) (width 0.2) (layer "F.Cu") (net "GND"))
 (segment (start 103.11 70.21) (end 103.11 85.71) (width 0.2) (layer "F.Cu") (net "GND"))
 (segment (start 146.25 90.54) (end 163.938 72.852) (width 0.2) (layer "F.Cu") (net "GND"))
 (segment (start 103.11 85.71) (end 112.11 94.71) (width 0.2) (layer "F.Cu") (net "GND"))
 (segment (start 163.938 66.402) (end 165 65.34) (width 0.2) (layer "F.Cu") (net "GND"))
 (segment (start 126.04 94.71) (end 134.134 86.616) (width 0.2) (layer "F.Cu") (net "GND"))
 (segment (start 134.134 86.616) (end 134.134 85.749) (width 0.2) (layer "F.Cu") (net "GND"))
 (segment (start 112.11 94.71) (end 126.04 94.71) (width 0.2) (layer "F.Cu") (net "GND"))
 (segment (start 103.11 70.21) (end 116.82 56.5) (width 0.2) (layer "F.Cu") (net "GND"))
 (segment (start 116.82 56.5) (end 126.63 56.5) (width 0.2) (layer "F.Cu") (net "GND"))
 (segment (start 134.134 85.749) (end 135.985 87.6) (width 0.2) (layer "B.Cu") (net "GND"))
 (segment (start 147.4 86.85) (end 147.4 89.39) (width 0.2) (layer "B.Cu") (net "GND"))
 (segment (start 145.1 86.85) (end 147.4 86.85) (width 0.2) (layer "B.Cu") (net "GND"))
 (segment (start 135.985 87.6) (end 144.35 87.6) (width 0.2) (layer "B.Cu") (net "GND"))
 (segment (start 147.4 89.39) (end 146.25 90.54) (width 0.2) (layer "B.Cu") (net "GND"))
 (segment (start 144.35 87.6) (end 145.1 86.85) (width 0.2) (layer "B.Cu") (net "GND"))
 (segment (start 167.351 66.60663) (end 166.07763 67.88) (width 0.2) (layer "F.Cu") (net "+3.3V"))
 (segment (start 134.5 56.25) (end 134.25 56.5) (width 0.2) (layer "F.Cu") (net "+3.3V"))
 (segment (start 164.560105 64.278) (end 167.090214 64.278) (width 0.2) (layer "F.Cu") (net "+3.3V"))
 (segment (start 166.07763 67.88) (end 165 67.88) (width 0.2) (layer "F.Cu") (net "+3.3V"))
 (segment (start 167.351 64.538786) (end 167.351 66.60663) (width 0.2) (layer "F.Cu") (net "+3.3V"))
 (segment (start 134.5 50.5) (end 134.5 56.25) (width 0.2) (layer "F.Cu") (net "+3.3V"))
 (segment (start 163.538 65.300105) (end 164.560105 64.278) (width 0.2) (layer "F.Cu") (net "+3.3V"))
 (segment (start 163.538 70.712) (end 163.538 65.300105) (width 0.2) (layer "F.Cu") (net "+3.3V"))
 (segment (start 146.25 88) (end 163.538 70.712) (width 0.2) (layer "F.Cu") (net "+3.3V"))
 (segment (start 167.090214 64.278) (end 167.351 64.538786) (width 0.2) (layer "F.Cu") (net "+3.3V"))
 (segment (start 131.594 85.749) (end 133.845 88) (width 0.2) (layer "B.Cu") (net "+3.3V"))
 (segment (start 134.25 83.093) (end 131.594 85.749) (width 0.2) (layer "B.Cu") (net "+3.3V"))
 (segment (start 133.845 88) (end 146.25 88) (width 0.2) (layer "B.Cu") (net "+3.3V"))
 (segment (start 134.25 56.5) (end 134.25 83.093) (width 0.2) (layer "B.Cu") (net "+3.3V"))
 (segment (start 145.1 77.007786) (end 149.147786 72.96) (width 0.2) (layer "F.Cu") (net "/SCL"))
 (segment (start 145.1 91.93) (end 145.1 77.007786) (width 0.2) (layer "F.Cu") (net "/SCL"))
 (segment (start 149.147786 72.96) (end 149.76 72.96) (width 0.2) (layer "F.Cu") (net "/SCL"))
 (segment (start 146.25 93.08) (end 145.1 91.93) (width 0.2) (layer "F.Cu") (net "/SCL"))
 (segment (start 136.385 93.08) (end 129.054 85.749) (width 0.2) (layer "B.Cu") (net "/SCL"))
 (segment (start 146.25 93.08) (end 136.385 93.08) (width 0.2) (layer "B.Cu") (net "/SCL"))
 (segment (start 150.822 76.562) (end 149.76 75.5) (width 0.2) (layer "F.Cu") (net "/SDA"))
 (segment (start 150.822 81.678) (end 150.822 76.562) (width 0.2) (layer "F.Cu") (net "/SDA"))
 (segment (start 146.25 95.62) (end 149.75 92.12) (width 0.2) (layer "F.Cu") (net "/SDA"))
 (segment (start 150.25 82.25) (end 150.822 81.678) (width 0.2) (layer "F.Cu") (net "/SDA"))
 (segment (start 149.75 92.12) (end 149.75 90.75) (width 0.2) (layer "F.Cu") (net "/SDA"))
 (via (at 150.25 82.25) (size 0.6) (drill 0.3) (layers "F.Cu" "B.Cu") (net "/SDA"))
 (via (at 149.75 90.75) (size 0.6) (drill 0.3) (layers "F.Cu" "B.Cu") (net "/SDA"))
 (segment (start 149.75 90.75) (end 149.75 82.75) (width 0.2) (layer "B.Cu") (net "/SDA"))
 (segment (start 149.75 82.75) (end 150.25 82.25) (width 0.2) (layer "B.Cu") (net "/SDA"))
 (segment (start 146.25 95.62) (end 136.385 95.62) (width 0.2) (layer "B.Cu") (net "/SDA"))
 (segment (start 136.385 95.62) (end 126.514 85.749) (width 0.2) (layer "B.Cu") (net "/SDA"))
 (segment (start 109.46 67.67) (end 149.55 67.67) (width 0.2) (layer "F.Cu") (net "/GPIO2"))
 (segment (start 149.55 67.67) (end 149.76 67.88) (width 0.2) (layer "F.Cu") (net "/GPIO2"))
 (segment (start 126.88 50.5) (end 126.88 51.67) (width 0.2) (layer "F.Cu") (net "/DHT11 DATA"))
 (segment (start 131.71 56.5) (end 140.55 65.34) (width 0.2) (layer "F.Cu") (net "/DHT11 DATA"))
 (segment (start 140.55 65.34) (end 149.76 65.34) (width 0.2) (layer "F.Cu") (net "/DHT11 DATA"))
 (segment (start 126.88 51.67) (end 131.71 56.5) (width 0.2) (layer "F.Cu") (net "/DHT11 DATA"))
 (segment (start 140.21 70.42) (end 149.76 70.42) (width 0.2) (layer "F.Cu") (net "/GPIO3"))
 (segment (start 118.46 92.17) (end 140.21 70.42) (width 0.2) (layer "F.Cu") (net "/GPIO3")))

